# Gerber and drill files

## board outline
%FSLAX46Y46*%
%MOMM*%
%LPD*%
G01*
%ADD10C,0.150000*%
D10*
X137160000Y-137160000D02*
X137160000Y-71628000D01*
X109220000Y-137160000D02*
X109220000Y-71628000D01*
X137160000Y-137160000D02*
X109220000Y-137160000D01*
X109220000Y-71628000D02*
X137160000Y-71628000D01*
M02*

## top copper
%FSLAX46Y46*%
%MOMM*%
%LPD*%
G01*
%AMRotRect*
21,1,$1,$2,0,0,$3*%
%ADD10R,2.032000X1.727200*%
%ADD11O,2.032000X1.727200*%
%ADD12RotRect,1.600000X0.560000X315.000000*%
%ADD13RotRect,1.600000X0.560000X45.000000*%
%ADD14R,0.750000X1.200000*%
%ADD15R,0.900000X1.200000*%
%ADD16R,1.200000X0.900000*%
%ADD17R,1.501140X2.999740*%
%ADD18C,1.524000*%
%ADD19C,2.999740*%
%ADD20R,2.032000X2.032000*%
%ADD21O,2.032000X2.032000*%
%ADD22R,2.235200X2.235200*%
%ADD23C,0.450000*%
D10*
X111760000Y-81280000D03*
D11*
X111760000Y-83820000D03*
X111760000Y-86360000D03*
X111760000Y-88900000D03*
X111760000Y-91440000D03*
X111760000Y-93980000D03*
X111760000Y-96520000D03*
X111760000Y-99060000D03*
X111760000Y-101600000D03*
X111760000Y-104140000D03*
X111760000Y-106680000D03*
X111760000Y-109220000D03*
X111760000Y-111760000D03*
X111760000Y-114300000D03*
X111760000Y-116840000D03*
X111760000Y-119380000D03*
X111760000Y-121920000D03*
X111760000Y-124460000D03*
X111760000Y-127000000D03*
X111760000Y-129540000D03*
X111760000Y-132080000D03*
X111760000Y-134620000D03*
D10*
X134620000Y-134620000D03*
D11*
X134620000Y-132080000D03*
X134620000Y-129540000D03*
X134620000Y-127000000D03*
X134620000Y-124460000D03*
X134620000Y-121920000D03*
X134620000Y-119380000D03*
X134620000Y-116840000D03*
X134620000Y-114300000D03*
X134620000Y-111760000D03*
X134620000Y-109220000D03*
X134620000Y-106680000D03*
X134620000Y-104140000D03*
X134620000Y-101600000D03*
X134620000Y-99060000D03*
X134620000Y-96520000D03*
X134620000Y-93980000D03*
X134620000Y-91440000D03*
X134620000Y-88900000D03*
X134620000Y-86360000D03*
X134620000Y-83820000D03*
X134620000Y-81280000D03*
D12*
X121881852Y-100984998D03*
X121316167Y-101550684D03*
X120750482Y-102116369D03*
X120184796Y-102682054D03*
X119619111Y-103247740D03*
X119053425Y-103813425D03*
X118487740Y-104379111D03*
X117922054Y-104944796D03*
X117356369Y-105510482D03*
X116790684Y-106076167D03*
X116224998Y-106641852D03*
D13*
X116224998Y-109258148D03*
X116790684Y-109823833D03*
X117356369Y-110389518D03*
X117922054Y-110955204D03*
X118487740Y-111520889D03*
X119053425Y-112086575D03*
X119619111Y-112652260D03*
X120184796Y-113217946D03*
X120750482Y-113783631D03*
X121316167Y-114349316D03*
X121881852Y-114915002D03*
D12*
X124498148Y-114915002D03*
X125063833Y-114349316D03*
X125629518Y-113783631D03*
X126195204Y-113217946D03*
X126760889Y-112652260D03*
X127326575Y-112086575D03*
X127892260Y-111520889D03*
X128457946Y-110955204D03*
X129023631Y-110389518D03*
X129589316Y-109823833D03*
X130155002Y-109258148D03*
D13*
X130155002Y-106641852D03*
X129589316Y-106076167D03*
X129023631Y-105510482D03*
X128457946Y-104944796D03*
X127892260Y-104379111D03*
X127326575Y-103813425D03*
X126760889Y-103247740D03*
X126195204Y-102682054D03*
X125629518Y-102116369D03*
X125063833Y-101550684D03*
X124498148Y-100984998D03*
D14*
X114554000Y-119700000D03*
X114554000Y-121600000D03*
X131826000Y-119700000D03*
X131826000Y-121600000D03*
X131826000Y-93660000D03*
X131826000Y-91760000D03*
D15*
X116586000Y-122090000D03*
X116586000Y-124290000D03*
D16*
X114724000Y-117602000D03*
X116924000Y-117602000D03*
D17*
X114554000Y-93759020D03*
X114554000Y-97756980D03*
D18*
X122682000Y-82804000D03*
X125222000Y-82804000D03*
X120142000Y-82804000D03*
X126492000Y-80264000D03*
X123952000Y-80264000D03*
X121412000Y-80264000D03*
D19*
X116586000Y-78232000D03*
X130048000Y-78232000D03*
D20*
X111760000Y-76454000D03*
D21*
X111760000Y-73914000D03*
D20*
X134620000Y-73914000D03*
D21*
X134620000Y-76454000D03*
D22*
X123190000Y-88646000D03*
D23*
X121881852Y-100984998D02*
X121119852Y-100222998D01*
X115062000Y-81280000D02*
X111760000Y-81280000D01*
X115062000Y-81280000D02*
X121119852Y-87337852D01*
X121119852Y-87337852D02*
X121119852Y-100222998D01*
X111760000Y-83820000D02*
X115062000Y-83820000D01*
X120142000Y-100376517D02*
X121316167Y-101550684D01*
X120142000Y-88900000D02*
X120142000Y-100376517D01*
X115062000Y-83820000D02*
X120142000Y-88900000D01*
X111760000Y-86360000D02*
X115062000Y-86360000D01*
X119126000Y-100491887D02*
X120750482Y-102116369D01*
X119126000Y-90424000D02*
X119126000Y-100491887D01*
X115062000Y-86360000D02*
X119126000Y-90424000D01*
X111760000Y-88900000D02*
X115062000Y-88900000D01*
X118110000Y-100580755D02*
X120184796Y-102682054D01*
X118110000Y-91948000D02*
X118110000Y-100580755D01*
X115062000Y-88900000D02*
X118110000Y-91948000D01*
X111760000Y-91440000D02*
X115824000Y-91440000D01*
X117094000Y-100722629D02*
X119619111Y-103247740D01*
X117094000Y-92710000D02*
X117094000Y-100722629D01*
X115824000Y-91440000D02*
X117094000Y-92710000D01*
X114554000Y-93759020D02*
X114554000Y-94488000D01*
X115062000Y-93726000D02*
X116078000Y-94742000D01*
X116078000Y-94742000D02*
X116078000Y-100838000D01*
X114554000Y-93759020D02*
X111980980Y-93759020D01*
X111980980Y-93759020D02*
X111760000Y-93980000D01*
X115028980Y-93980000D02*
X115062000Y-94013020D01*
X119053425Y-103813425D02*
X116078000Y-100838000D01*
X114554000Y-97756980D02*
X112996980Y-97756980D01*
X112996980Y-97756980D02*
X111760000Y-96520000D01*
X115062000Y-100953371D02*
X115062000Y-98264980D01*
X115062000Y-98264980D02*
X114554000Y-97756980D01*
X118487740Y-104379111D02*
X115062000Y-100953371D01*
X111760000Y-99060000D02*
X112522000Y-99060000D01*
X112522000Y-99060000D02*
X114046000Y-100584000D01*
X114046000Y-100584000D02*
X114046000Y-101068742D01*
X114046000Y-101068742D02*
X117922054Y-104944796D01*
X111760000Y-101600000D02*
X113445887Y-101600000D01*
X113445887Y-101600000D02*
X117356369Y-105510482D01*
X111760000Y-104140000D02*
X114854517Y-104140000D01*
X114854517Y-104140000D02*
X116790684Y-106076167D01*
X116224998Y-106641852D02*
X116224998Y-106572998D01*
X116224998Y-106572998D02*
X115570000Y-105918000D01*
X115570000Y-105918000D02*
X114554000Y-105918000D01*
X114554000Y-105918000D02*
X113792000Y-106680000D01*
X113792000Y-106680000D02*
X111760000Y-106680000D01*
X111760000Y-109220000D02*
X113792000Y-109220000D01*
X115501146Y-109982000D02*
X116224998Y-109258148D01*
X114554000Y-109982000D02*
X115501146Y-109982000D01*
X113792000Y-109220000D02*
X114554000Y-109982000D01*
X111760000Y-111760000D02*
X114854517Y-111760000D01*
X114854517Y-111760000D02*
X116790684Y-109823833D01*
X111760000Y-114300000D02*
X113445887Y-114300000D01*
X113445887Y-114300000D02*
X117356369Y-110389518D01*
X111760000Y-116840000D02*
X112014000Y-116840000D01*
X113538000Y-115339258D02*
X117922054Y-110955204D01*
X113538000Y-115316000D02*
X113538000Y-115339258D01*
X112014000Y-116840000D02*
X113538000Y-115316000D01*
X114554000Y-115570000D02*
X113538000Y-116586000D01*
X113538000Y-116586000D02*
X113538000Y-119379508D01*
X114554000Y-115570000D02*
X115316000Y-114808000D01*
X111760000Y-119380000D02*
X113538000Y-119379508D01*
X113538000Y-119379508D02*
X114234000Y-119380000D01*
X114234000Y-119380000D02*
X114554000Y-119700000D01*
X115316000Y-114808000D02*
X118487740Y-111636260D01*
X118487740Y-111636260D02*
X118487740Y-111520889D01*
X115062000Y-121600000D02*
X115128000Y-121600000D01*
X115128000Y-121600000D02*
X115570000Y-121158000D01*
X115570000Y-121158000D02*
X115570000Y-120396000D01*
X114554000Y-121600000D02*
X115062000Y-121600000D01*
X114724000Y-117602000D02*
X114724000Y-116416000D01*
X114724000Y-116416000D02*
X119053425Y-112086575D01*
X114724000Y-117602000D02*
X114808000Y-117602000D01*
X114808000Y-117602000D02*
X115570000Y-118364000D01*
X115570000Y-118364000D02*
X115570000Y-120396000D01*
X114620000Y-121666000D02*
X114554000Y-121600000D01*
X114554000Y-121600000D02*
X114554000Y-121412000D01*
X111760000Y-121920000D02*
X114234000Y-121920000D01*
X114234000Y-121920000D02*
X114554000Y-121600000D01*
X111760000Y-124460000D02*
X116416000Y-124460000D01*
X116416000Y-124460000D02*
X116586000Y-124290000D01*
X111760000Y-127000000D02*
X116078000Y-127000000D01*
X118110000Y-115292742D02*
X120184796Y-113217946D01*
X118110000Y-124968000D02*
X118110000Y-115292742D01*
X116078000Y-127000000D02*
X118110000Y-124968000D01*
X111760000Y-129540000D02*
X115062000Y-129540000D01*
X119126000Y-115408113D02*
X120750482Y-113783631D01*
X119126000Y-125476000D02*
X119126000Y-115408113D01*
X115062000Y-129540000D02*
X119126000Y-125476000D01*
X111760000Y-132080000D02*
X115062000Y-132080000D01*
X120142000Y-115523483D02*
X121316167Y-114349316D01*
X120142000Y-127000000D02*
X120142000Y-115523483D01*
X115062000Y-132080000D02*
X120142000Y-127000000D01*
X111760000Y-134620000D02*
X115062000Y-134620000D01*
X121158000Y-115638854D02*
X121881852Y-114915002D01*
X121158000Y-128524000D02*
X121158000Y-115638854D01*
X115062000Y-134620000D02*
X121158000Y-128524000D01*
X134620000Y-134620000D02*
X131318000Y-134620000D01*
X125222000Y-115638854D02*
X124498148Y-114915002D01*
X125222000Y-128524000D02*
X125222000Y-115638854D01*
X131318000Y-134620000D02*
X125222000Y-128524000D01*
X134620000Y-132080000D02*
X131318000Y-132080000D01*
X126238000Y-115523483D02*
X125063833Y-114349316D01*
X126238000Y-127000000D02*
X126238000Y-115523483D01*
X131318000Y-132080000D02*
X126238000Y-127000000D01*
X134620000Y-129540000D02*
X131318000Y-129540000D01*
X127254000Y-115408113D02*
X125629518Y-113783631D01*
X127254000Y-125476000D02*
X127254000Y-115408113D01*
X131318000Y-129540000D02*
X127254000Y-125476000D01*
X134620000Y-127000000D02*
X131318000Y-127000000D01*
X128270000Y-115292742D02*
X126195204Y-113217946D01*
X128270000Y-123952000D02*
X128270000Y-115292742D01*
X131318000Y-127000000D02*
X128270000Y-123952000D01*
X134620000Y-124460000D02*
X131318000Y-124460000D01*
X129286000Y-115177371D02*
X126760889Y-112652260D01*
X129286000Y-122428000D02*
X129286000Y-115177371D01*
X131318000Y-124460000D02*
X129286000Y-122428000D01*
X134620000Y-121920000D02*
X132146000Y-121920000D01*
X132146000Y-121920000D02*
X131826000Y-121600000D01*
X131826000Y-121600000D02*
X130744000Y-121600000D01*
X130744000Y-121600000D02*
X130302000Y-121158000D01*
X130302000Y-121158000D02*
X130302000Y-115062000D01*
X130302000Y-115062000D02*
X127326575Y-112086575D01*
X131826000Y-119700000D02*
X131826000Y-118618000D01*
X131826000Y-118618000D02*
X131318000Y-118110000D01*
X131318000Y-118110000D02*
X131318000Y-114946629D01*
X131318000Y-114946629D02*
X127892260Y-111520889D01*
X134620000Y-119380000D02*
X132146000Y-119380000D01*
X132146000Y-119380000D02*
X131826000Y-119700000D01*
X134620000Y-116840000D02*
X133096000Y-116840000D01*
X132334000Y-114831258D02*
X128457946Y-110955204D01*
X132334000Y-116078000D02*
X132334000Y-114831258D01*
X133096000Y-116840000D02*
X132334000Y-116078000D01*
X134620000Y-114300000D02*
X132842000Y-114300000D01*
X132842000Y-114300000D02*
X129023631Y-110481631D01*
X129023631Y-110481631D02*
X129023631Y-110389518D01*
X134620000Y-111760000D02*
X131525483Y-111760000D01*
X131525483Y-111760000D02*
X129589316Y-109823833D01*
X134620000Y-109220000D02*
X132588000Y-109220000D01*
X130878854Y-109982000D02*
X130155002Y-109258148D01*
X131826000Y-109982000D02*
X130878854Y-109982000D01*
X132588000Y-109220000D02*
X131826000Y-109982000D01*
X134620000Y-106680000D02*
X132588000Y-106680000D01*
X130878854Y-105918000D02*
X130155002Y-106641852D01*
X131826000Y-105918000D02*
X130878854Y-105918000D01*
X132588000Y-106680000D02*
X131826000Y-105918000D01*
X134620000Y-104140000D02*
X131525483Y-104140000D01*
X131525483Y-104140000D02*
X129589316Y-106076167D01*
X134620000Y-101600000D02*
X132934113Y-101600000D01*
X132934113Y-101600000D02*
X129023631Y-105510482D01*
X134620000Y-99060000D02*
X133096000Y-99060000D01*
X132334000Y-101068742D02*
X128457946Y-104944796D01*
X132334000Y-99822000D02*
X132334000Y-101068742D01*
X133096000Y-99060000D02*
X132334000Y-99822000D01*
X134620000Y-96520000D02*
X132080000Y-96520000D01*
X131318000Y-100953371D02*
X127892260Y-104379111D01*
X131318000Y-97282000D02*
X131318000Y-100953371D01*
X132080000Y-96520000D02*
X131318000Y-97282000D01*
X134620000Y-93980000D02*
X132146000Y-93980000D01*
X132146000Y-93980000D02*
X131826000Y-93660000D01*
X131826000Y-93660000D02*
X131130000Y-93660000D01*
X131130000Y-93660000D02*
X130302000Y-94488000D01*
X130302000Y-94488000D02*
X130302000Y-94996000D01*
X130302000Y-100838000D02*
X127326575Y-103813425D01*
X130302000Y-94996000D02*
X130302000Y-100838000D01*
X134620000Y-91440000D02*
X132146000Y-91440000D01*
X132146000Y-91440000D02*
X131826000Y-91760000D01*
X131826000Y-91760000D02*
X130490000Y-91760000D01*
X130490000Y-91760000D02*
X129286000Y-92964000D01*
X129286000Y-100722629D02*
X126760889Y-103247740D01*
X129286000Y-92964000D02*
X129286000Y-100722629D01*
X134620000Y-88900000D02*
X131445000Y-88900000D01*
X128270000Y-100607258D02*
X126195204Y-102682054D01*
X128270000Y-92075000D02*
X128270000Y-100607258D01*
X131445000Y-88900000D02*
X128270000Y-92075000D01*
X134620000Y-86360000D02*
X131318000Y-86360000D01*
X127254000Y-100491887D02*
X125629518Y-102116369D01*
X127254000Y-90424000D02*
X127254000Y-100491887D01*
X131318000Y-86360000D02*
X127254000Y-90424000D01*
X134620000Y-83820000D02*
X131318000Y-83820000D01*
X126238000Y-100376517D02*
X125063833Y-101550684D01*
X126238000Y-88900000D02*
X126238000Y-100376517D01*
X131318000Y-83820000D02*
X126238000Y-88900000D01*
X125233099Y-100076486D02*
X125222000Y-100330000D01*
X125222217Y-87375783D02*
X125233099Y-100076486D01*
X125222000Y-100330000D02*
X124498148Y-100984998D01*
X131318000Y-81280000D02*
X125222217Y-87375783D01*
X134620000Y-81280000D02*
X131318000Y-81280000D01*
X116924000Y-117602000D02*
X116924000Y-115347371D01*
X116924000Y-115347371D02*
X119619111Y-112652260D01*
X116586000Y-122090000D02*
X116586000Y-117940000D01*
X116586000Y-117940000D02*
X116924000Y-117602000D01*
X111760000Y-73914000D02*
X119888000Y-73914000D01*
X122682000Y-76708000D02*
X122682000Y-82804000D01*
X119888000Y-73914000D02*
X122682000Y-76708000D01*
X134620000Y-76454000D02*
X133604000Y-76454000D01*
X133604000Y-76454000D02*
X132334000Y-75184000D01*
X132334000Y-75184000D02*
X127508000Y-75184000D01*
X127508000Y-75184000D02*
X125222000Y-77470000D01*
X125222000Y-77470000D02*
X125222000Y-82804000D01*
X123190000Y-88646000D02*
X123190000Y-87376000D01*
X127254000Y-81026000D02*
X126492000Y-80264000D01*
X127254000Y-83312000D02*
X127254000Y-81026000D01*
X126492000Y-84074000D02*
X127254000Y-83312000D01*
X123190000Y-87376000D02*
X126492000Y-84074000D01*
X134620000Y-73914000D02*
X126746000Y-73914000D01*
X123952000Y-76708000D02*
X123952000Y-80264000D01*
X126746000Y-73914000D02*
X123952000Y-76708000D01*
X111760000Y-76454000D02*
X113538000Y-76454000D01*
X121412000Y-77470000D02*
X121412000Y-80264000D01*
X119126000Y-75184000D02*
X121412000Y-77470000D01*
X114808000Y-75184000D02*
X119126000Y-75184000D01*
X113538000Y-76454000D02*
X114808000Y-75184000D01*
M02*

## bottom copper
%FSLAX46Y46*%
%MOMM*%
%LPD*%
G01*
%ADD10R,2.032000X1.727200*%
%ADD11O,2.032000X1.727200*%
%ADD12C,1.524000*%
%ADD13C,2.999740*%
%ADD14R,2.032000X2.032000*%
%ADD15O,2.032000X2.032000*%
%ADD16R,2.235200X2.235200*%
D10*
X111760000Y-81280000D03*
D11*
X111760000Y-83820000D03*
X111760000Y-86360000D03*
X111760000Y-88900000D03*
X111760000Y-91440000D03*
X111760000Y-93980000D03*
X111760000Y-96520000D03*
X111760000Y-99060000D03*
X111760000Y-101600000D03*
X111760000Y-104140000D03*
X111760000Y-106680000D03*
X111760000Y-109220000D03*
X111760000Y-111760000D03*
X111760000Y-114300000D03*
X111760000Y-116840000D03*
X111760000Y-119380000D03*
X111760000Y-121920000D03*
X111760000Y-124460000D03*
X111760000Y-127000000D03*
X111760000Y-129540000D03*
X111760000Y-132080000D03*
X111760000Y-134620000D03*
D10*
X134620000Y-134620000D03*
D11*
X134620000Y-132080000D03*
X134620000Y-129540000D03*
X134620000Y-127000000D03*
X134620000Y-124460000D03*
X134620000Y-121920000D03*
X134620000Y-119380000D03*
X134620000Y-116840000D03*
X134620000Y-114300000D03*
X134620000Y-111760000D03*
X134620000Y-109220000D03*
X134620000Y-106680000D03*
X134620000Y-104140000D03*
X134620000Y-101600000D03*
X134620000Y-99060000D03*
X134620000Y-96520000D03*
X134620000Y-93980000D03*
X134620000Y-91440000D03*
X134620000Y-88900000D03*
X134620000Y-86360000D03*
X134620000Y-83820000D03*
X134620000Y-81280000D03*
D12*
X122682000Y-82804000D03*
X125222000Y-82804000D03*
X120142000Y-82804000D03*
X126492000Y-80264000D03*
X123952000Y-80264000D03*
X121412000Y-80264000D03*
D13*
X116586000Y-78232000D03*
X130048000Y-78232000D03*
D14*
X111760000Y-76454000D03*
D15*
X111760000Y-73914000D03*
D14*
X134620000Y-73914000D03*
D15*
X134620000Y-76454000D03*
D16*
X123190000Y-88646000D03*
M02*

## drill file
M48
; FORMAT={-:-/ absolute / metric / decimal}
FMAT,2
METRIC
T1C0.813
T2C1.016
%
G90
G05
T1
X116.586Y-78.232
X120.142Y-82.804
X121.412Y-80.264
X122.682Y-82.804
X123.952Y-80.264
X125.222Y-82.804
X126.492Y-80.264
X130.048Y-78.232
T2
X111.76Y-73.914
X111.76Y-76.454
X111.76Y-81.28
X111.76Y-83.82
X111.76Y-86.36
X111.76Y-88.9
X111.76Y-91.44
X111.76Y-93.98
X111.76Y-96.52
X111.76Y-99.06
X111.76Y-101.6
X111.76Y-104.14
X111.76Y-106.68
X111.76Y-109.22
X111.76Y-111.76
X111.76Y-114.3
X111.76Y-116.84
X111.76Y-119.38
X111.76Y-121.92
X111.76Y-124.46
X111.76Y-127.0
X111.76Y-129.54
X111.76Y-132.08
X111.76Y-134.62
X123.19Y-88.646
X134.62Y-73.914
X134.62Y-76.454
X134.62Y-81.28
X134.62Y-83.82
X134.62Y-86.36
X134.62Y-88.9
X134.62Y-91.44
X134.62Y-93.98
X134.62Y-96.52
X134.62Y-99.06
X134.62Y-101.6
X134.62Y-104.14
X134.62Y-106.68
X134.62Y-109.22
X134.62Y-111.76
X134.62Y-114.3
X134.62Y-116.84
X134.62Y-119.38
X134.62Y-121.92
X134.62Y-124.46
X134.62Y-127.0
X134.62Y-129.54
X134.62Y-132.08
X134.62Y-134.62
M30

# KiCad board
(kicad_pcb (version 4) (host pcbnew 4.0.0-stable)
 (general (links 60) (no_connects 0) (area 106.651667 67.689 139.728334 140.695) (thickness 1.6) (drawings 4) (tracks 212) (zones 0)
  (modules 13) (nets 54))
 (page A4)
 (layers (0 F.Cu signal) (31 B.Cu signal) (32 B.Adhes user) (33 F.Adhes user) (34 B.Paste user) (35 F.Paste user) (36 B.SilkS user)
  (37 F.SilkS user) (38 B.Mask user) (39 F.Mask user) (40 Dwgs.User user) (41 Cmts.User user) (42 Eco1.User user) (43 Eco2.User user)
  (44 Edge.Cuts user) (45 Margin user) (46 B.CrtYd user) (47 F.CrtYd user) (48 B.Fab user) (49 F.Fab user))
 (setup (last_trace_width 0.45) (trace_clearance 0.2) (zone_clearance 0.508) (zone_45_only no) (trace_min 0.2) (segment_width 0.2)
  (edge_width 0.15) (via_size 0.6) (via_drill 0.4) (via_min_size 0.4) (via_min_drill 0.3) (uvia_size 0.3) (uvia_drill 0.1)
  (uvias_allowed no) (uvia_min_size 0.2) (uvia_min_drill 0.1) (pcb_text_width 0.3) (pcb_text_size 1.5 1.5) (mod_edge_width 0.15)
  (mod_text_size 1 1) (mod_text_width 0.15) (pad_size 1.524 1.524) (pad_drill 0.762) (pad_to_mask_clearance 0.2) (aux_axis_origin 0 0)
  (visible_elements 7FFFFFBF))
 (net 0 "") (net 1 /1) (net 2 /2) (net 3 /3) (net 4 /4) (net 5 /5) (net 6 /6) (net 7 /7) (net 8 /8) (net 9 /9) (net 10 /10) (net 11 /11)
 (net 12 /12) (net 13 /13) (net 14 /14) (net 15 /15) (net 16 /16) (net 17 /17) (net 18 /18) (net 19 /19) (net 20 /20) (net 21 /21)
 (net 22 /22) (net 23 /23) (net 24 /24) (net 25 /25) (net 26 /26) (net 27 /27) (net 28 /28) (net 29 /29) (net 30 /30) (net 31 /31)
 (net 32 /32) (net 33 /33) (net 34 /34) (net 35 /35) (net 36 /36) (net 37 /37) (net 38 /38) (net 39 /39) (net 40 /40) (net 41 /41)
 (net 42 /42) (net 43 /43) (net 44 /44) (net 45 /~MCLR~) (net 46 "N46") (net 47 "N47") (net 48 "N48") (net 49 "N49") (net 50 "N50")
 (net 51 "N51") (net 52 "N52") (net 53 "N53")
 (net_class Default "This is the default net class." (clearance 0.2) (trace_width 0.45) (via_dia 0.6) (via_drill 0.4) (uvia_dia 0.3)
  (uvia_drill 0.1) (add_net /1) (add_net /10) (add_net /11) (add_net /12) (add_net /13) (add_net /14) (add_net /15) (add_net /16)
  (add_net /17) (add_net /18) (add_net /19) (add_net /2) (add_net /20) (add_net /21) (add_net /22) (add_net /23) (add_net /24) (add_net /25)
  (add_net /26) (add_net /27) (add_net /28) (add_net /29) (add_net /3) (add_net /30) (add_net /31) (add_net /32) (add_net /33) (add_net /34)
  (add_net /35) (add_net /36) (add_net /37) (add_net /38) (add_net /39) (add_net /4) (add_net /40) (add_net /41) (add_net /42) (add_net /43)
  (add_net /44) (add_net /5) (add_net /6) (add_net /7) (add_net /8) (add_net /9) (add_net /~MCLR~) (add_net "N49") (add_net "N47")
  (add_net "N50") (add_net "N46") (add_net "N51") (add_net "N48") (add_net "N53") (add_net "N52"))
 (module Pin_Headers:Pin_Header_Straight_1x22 (layer B.Cu) (at 111.76 81.28 180)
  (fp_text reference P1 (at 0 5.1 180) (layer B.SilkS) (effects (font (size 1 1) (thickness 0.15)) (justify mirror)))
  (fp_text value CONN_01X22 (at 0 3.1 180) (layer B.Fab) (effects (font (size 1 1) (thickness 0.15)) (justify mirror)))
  (pad 1 thru_hole rect (at 0 0 180) (size 2.032 1.7272) (drill 1.016) (layers *.Cu *.Mask B.SilkS) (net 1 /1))
  (pad 2 thru_hole oval (at 0 -2.54 180) (size 2.032 1.7272) (drill 1.016) (layers *.Cu *.Mask B.SilkS) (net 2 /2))
  (pad 3 thru_hole oval (at 0 -5.08 180) (size 2.032 1.7272) (drill 1.016) (layers *.Cu *.Mask B.SilkS) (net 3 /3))
  (pad 4 thru_hole oval (at 0 -7.62 180) (size 2.032 1.7272) (drill 1.016) (layers *.Cu *.Mask B.SilkS) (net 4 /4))
  (pad 5 thru_hole oval (at 0 -10.16 180) (size 2.032 1.7272) (drill 1.016) (layers *.Cu *.Mask B.SilkS) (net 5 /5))
  (pad 6 thru_hole oval (at 0 -12.7 180) (size 2.032 1.7272) (drill 1.016) (layers *.Cu *.Mask B.SilkS) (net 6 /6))
  (pad 7 thru_hole oval (at 0 -15.24 180) (size 2.032 1.7272) (drill 1.016) (layers *.Cu *.Mask B.SilkS) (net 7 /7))
  (pad 8 thru_hole oval (at 0 -17.78 180) (size 2.032 1.7272) (drill 1.016) (layers *.Cu *.Mask B.SilkS) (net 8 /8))
  (pad 9 thru_hole oval (at 0 -20.32 180) (size 2.032 1.7272) (drill 1.016) (layers *.Cu *.Mask B.SilkS) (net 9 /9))
  (pad 10 thru_hole oval (at 0 -22.86 180) (size 2.032 1.7272) (drill 1.016) (layers *.Cu *.Mask B.SilkS) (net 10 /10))
  (pad 11 thru_hole oval (at 0 -25.4 180) (size 2.032 1.7272) (drill 1.016) (layers *.Cu *.Mask B.SilkS) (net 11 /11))
  (pad 12 thru_hole oval (at 0 -27.94 180) (size 2.032 1.7272) (drill 1.016) (layers *.Cu *.Mask B.SilkS) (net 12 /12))
  (pad 13 thru_hole oval (at 0 -30.48 180) (size 2.032 1.7272) (drill 1.016) (layers *.Cu *.Mask B.SilkS) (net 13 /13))
  (pad 14 thru_hole oval (at 0 -33.02 180) (size 2.032 1.7272) (drill 1.016) (layers *.Cu *.Mask B.SilkS) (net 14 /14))
  (pad 15 thru_hole oval (at 0 -35.56 180) (size 2.032 1.7272) (drill 1.016) (layers *.Cu *.Mask B.SilkS) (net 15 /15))
  (pad 16 thru_hole oval (at 0 -38.1 180) (size 2.032 1.7272) (drill 1.016) (layers *.Cu *.Mask B.SilkS) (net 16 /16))
  (pad 17 thru_hole oval (at 0 -40.64 180) (size 2.032 1.7272) (drill 1.016) (layers *.Cu *.Mask B.SilkS) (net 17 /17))
  (pad 18 thru_hole oval (at 0 -43.18 180) (size 2.032 1.7272) (drill 1.016) (layers *.Cu *.Mask B.SilkS) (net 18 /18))
  (pad 19 thru_hole oval (at 0 -45.72 180) (size 2.032 1.7272) (drill 1.016) (layers *.Cu *.Mask B.SilkS) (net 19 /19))
  (pad 20 thru_hole oval (at 0 -48.26 180) (size 2.032 1.7272) (drill 1.016) (layers *.Cu *.Mask B.SilkS) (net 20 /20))
  (pad 21 thru_hole oval (at 0 -50.8 180) (size 2.032 1.7272) (drill 1.016) (layers *.Cu *.Mask B.SilkS) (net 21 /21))
  (pad 22 thru_hole oval (at 0 -53.34 180) (size 2.032 1.7272) (drill 1.016) (layers *.Cu *.Mask B.SilkS) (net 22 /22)))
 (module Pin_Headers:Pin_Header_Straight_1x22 (layer B.Cu) (at 134.62 134.62)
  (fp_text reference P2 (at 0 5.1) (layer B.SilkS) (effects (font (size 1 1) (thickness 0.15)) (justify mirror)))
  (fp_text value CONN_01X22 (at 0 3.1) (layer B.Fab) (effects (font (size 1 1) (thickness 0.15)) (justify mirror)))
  (pad 1 thru_hole rect (at 0 0) (size 2.032 1.7272) (drill 1.016) (layers *.Cu *.Mask B.SilkS) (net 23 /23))
  (pad 2 thru_hole oval (at 0 -2.54) (size 2.032 1.7272) (drill 1.016) (layers *.Cu *.Mask B.SilkS) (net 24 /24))
  (pad 3 thru_hole oval (at 0 -5.08) (size 2.032 1.7272) (drill 1.016) (layers *.Cu *.Mask B.SilkS) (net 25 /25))
  (pad 4 thru_hole oval (at 0 -7.62) (size 2.032 1.7272) (drill 1.016) (layers *.Cu *.Mask B.SilkS) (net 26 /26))
  (pad 5 thru_hole oval (at 0 -10.16) (size 2.032 1.7272) (drill 1.016) (layers *.Cu *.Mask B.SilkS) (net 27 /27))
  (pad 6 thru_hole oval (at 0 -12.7) (size 2.032 1.7272) (drill 1.016) (layers *.Cu *.Mask B.SilkS) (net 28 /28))
  (pad 7 thru_hole oval (at 0 -15.24) (size 2.032 1.7272) (drill 1.016) (layers *.Cu *.Mask B.SilkS) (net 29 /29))
  (pad 8 thru_hole oval (at 0 -17.78) (size 2.032 1.7272) (drill 1.016) (layers *.Cu *.Mask B.SilkS) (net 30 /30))
  (pad 9 thru_hole oval (at 0 -20.32) (size 2.032 1.7272) (drill 1.016) (layers *.Cu *.Mask B.SilkS) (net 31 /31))
  (pad 10 thru_hole oval (at 0 -22.86) (size 2.032 1.7272) (drill 1.016) (layers *.Cu *.Mask B.SilkS) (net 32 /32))
  (pad 11 thru_hole oval (at 0 -25.4) (size 2.032 1.7272) (drill 1.016) (layers *.Cu *.Mask B.SilkS) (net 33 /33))
  (pad 12 thru_hole oval (at 0 -27.94) (size 2.032 1.7272) (drill 1.016) (layers *.Cu *.Mask B.SilkS) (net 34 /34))
  (pad 13 thru_hole oval (at 0 -30.48) (size 2.032 1.7272) (drill 1.016) (layers *.Cu *.Mask B.SilkS) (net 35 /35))
  (pad 14 thru_hole oval (at 0 -33.02) (size 2.032 1.7272) (drill 1.016) (layers *.Cu *.Mask B.SilkS) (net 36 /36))
  (pad 15 thru_hole oval (at 0 -35.56) (size 2.032 1.7272) (drill 1.016) (layers *.Cu *.Mask B.SilkS) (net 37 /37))
  (pad 16 thru_hole oval (at 0 -38.1) (size 2.032 1.7272) (drill 1.016) (layers *.Cu *.Mask B.SilkS) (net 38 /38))
  (pad 17 thru_hole oval (at 0 -40.64) (size 2.032 1.7272) (drill 1.016) (layers *.Cu *.Mask B.SilkS) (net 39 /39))
  (pad 18 thru_hole oval (at 0 -43.18) (size 2.032 1.7272) (drill 1.016) (layers *.Cu *.Mask B.SilkS) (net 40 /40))
  (pad 19 thru_hole oval (at 0 -45.72) (size 2.032 1.7272) (drill 1.016) (layers *.Cu *.Mask B.SilkS) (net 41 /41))
  (pad 20 thru_hole oval (at 0 -48.26) (size 2.032 1.7272) (drill 1.016) (layers *.Cu *.Mask B.SilkS) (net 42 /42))
  (pad 21 thru_hole oval (at 0 -50.8) (size 2.032 1.7272) (drill 1.016) (layers *.Cu *.Mask B.SilkS) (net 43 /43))
  (pad 22 thru_hole oval (at 0 -53.34) (size 2.032 1.7272) (drill 1.016) (layers *.Cu *.Mask B.SilkS) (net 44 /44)))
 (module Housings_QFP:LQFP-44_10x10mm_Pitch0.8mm (layer F.Cu) (at 123.19 107.95 315)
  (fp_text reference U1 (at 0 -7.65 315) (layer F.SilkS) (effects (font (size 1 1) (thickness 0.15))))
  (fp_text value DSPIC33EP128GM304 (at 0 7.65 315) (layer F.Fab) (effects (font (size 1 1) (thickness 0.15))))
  (pad 1 smd rect (at -5.85 -4 315) (size 1.6 0.56) (layers F.Cu F.Paste F.Mask) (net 1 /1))
  (pad 2 smd rect (at -5.85 -3.2 315) (size 1.6 0.56) (layers F.Cu F.Paste F.Mask) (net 2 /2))
  (pad 3 smd rect (at -5.85 -2.4 315) (size 1.6 0.56) (layers F.Cu F.Paste F.Mask) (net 3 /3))
  (pad 4 smd rect (at -5.85 -1.6 315) (size 1.6 0.56) (layers F.Cu F.Paste F.Mask) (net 4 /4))
  (pad 5 smd rect (at -5.85 -0.8 315) (size 1.6 0.56) (layers F.Cu F.Paste F.Mask) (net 5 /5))
  (pad 6 smd rect (at -5.85 0 315) (size 1.6 0.56) (layers F.Cu F.Paste F.Mask) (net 6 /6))
  (pad 7 smd rect (at -5.85 0.8 315) (size 1.6 0.56) (layers F.Cu F.Paste F.Mask) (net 7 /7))
  (pad 8 smd rect (at -5.85 1.6 315) (size 1.6 0.56) (layers F.Cu F.Paste F.Mask) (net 8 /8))
  (pad 9 smd rect (at -5.85 2.4 315) (size 1.6 0.56) (layers F.Cu F.Paste F.Mask) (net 9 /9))
  (pad 10 smd rect (at -5.85 3.2 315) (size 1.6 0.56) (layers F.Cu F.Paste F.Mask) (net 10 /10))
  (pad 11 smd rect (at -5.85 4 315) (size 1.6 0.56) (layers F.Cu F.Paste F.Mask) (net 11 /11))
  (pad 12 smd rect (at -4 5.85 45) (size 1.6 0.56) (layers F.Cu F.Paste F.Mask) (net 12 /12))
  (pad 13 smd rect (at -3.2 5.85 45) (size 1.6 0.56) (layers F.Cu F.Paste F.Mask) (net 13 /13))
  (pad 14 smd rect (at -2.4 5.85 45) (size 1.6 0.56) (layers F.Cu F.Paste F.Mask) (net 14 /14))
  (pad 15 smd rect (at -1.6 5.85 45) (size 1.6 0.56) (layers F.Cu F.Paste F.Mask) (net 15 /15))
  (pad 16 smd rect (at -0.8 5.85 45) (size 1.6 0.56) (layers F.Cu F.Paste F.Mask) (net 16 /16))
  (pad 17 smd rect (at 0 5.85 45) (size 1.6 0.56) (layers F.Cu F.Paste F.Mask) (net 17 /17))
  (pad 18 smd rect (at 0.8 5.85 45) (size 1.6 0.56) (layers F.Cu F.Paste F.Mask) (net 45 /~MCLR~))
  (pad 19 smd rect (at 1.6 5.85 45) (size 1.6 0.56) (layers F.Cu F.Paste F.Mask) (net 19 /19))
  (pad 20 smd rect (at 2.4 5.85 45) (size 1.6 0.56) (layers F.Cu F.Paste F.Mask) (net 20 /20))
  (pad 21 smd rect (at 3.2 5.85 45) (size 1.6 0.56) (layers F.Cu F.Paste F.Mask) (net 21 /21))
  (pad 22 smd rect (at 4 5.85 45) (size 1.6 0.56) (layers F.Cu F.Paste F.Mask) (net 22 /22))
  (pad 23 smd rect (at 5.85 4 315) (size 1.6 0.56) (layers F.Cu F.Paste F.Mask) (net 23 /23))
  (pad 24 smd rect (at 5.85 3.2 315) (size 1.6 0.56) (layers F.Cu F.Paste F.Mask) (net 24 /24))
  (pad 25 smd rect (at 5.85 2.4 315) (size 1.6 0.56) (layers F.Cu F.Paste F.Mask) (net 25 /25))
  (pad 26 smd rect (at 5.85 1.6 315) (size 1.6 0.56) (layers F.Cu F.Paste F.Mask) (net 26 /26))
  (pad 27 smd rect (at 5.85 0.8 315) (size 1.6 0.56) (layers F.Cu F.Paste F.Mask) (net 27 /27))
  (pad 28 smd rect (at 5.85 0 315) (size 1.6 0.56) (layers F.Cu F.Paste F.Mask) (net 28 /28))
  (pad 29 smd rect (at 5.85 -0.8 315) (size 1.6 0.56) (layers F.Cu F.Paste F.Mask) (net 29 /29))
  (pad 30 smd rect (at 5.85 -1.6 315) (size 1.6 0.56) (layers F.Cu F.Paste F.Mask) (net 30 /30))
  (pad 31 smd rect (at 5.85 -2.4 315) (size 1.6 0.56) (layers F.Cu F.Paste F.Mask) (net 31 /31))
  (pad 32 smd rect (at 5.85 -3.2 315) (size 1.6 0.56) (layers F.Cu F.Paste F.Mask) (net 32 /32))
  (pad 33 smd rect (at 5.85 -4 315) (size 1.6 0.56) (layers F.Cu F.Paste F.Mask) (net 33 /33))
  (pad 34 smd rect (at 4 -5.85 45) (size 1.6 0.56) (layers F.Cu F.Paste F.Mask) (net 34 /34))
  (pad 35 smd rect (at 3.2 -5.85 45) (size 1.6 0.56) (layers F.Cu F.Paste F.Mask) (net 35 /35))
  (pad 36 smd rect (at 2.4 -5.85 45) (size 1.6 0.56) (layers F.Cu F.Paste F.Mask) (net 36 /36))
  (pad 37 smd rect (at 1.6 -5.85 45) (size 1.6 0.56) (layers F.Cu F.Paste F.Mask) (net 37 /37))
  (pad 38 smd rect (at 0.8 -5.85 45) (size 1.6 0.56) (layers F.Cu F.Paste F.Mask) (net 38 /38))
  (pad 39 smd rect (at 0 -5.85 45) (size 1.6 0.56) (layers F.Cu F.Paste F.Mask) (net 39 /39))
  (pad 40 smd rect (at -0.8 -5.85 45) (size 1.6 0.56) (layers F.Cu F.Paste F.Mask) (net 40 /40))
  (pad 41 smd rect (at -1.6 -5.85 45) (size 1.6 0.56) (layers F.Cu F.Paste F.Mask) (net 41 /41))
  (pad 42 smd rect (at -2.4 -5.85 45) (size 1.6 0.56) (layers F.Cu F.Paste F.Mask) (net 42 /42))
  (pad 43 smd rect (at -3.2 -5.85 45) (size 1.6 0.56) (layers F.Cu F.Paste F.Mask) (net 43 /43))
  (pad 44 smd rect (at -4 -5.85 45) (size 1.6 0.56) (layers F.Cu F.Paste F.Mask) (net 44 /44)))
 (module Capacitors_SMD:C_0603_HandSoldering (layer F.Cu) (at 114.554 120.65 270)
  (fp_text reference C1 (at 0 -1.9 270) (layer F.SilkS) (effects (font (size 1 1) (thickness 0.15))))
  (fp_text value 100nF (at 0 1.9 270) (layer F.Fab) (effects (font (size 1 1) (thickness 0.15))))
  (pad 1 smd rect (at -0.95 0 270) (size 1.2 0.75) (layers F.Cu F.Paste F.Mask) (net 16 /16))
  (pad 2 smd rect (at 0.95 0 270) (size 1.2 0.75) (layers F.Cu F.Paste F.Mask) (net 17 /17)))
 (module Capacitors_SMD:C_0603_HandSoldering (layer F.Cu) (at 131.826 120.65 270)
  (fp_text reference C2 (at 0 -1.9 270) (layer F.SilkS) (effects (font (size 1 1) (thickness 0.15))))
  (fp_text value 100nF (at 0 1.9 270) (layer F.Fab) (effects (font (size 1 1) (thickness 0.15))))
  (pad 1 smd rect (at -0.95 0 270) (size 1.2 0.75) (layers F.Cu F.Paste F.Mask) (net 29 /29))
  (pad 2 smd rect (at 0.95 0 270) (size 1.2 0.75) (layers F.Cu F.Paste F.Mask) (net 28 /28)))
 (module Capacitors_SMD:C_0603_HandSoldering (layer F.Cu) (at 131.826 92.71 90)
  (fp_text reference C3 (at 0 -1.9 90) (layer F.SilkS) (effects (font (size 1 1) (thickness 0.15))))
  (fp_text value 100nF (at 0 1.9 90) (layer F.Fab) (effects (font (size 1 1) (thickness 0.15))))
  (pad 1 smd rect (at -0.95 0 90) (size 1.2 0.75) (layers F.Cu F.Paste F.Mask) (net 39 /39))
  (pad 2 smd rect (at 0.95 0 90) (size 1.2 0.75) (layers F.Cu F.Paste F.Mask) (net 40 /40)))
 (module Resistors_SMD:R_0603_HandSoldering (layer F.Cu) (at 116.586 123.19 270)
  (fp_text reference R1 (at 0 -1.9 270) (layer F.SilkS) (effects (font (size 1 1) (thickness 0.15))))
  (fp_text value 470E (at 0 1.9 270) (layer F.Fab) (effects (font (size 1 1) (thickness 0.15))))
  (pad 1 smd rect (at -1.1 0 270) (size 1.2 0.9) (layers F.Cu F.Paste F.Mask) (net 45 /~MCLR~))
  (pad 2 smd rect (at 1.1 0 270) (size 1.2 0.9) (layers F.Cu F.Paste F.Mask) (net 18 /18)))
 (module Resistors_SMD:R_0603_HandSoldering (layer F.Cu) (at 115.824 117.602)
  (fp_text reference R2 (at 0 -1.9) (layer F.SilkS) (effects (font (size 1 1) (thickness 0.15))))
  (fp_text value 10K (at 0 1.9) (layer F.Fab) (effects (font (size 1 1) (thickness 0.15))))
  (pad 1 smd rect (at -1.1 0) (size 1.2 0.9) (layers F.Cu F.Paste F.Mask) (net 17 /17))
  (pad 2 smd rect (at 1.1 0) (size 1.2 0.9) (layers F.Cu F.Paste F.Mask) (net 45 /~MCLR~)))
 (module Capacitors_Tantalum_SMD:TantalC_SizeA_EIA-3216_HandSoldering (layer F.Cu) (at 114.554 95.758 90)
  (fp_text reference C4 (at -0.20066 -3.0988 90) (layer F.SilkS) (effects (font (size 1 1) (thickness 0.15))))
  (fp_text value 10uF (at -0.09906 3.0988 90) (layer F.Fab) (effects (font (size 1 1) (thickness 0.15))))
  (pad 2 smd rect (at 1.99898 0 90) (size 2.99974 1.50114) (layers F.Cu F.Paste F.Mask) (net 6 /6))
  (pad 1 smd rect (at -1.99898 0 90) (size 2.99974 1.50114) (layers F.Cu F.Paste F.Mask) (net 7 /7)))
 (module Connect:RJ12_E (layer F.Cu) (at 123.19 73.914 180)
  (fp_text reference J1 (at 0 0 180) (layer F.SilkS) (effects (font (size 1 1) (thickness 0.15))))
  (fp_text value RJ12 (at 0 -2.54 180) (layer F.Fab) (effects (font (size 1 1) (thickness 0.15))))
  (pad 4 thru_hole circle (at 0.508 -8.89 180) (size 1.524 1.524) (drill 0.8128) (layers *.Cu *.Mask F.SilkS) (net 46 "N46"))
  (pad 2 thru_hole circle (at -2.032 -8.89 180) (size 1.524 1.524) (drill 0.8128) (layers *.Cu *.Mask F.SilkS) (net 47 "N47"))
  (pad 6 thru_hole circle (at 3.048 -8.89 180) (size 1.524 1.524) (drill 0.8128) (layers *.Cu *.Mask F.SilkS) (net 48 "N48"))
  (pad 1 thru_hole circle (at -3.302 -6.35 180) (size 1.524 1.524) (drill 0.8128) (layers *.Cu *.Mask F.SilkS) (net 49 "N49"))
  (pad 3 thru_hole circle (at -0.762 -6.35 180) (size 1.524 1.524) (drill 0.8128) (layers *.Cu *.Mask F.SilkS) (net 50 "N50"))
  (pad 5 thru_hole circle (at 1.778 -6.35 180) (size 1.524 1.524) (drill 0.8128) (layers *.Cu *.Mask F.SilkS) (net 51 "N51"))
  (pad 8 thru_hole circle (at 6.604 -4.318 180) (size 2.99974 2.99974) (drill 0.8128) (layers *.Cu *.Mask F.SilkS) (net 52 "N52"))
  (pad 7 thru_hole circle (at -6.858 -4.318 180) (size 2.99974 2.99974) (drill 0.8128) (layers *.Cu *.Mask F.SilkS) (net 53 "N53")))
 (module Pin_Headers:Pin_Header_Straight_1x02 (layer F.Cu) (at 111.76 76.454 180)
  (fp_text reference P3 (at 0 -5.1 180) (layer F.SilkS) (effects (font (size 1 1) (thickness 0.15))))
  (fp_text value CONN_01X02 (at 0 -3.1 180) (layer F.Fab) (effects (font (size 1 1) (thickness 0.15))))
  (pad 1 thru_hole rect (at 0 0 180) (size 2.032 2.032) (drill 1.016) (layers *.Cu *.Mask F.SilkS) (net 51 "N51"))
  (pad 2 thru_hole oval (at 0 2.54 180) (size 2.032 2.032) (drill 1.016) (layers *.Cu *.Mask F.SilkS) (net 46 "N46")))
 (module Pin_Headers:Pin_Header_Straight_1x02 (layer F.Cu) (at 134.62 73.914)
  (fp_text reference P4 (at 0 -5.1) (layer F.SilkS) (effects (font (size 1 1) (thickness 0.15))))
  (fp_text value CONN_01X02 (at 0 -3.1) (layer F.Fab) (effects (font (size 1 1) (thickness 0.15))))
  (pad 1 thru_hole rect (at 0 0) (size 2.032 2.032) (drill 1.016) (layers *.Cu *.Mask F.SilkS) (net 50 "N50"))
  (pad 2 thru_hole oval (at 0 2.54) (size 2.032 2.032) (drill 1.016) (layers *.Cu *.Mask F.SilkS) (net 47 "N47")))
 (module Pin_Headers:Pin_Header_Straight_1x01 (layer F.Cu) (at 123.19 88.646)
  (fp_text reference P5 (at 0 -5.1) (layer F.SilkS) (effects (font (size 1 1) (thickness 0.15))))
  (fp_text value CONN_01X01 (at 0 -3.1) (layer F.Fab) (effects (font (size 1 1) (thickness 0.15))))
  (pad 1 thru_hole rect (at 0 0) (size 2.2352 2.2352) (drill 1.016) (layers *.Cu *.Mask F.SilkS) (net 49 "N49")))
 (gr_line (start 137.16 137.16) (end 137.16 71.628) (angle 90) (layer Edge.Cuts) (width 0.15))
 (gr_line (start 109.22 137.16) (end 109.22 71.628) (angle 90) (layer Edge.Cuts) (width 0.15))
 (gr_line (start 137.16 137.16) (end 109.22 137.16) (angle 90) (layer Edge.Cuts) (width 0.15))
 (gr_line (start 109.22 71.628) (end 137.16 71.628) (angle 90) (layer Edge.Cuts) (width 0.15))
 (segment (start 121.881852 100.984998) (end 121.119852 100.222998) (width 0.45) (layer F.Cu) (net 1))
 (segment (start 115.062 81.28) (end 111.76 81.28) (width 0.45) (layer F.Cu) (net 1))
 (segment (start 115.062 81.28) (end 121.119852 87.337852) (width 0.45) (layer F.Cu) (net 1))
 (segment (start 121.119852 87.337852) (end 121.119852 100.222998) (width 0.45) (layer F.Cu) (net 1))
 (segment (start 111.76 83.82) (end 115.062 83.82) (width 0.45) (layer F.Cu) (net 2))
 (segment (start 120.142 100.376517) (end 121.316167 101.550684) (width 0.45) (layer F.Cu) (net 2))
 (segment (start 120.142 88.9) (end 120.142 100.376517) (width 0.45) (layer F.Cu) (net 2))
 (segment (start 115.062 83.82) (end 120.142 88.9) (width 0.45) (layer F.Cu) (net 2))
 (segment (start 111.76 86.36) (end 115.062 86.36) (width 0.45) (layer F.Cu) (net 3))
 (segment (start 119.126 100.491887) (end 120.750482 102.116369) (width 0.45) (layer F.Cu) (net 3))
 (segment (start 119.126 90.424) (end 119.126 100.491887) (width 0.45) (layer F.Cu) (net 3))
 (segment (start 115.062 86.36) (end 119.126 90.424) (width 0.45) (layer F.Cu) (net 3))
 (segment (start 111.76 88.9) (end 115.062 88.9) (width 0.45) (layer F.Cu) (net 4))
 (segment (start 118.11 100.580755) (end 120.184796 102.682054) (width 0.45) (layer F.Cu) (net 4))
 (segment (start 118.11 91.948) (end 118.11 100.580755) (width 0.45) (layer F.Cu) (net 4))
 (segment (start 115.062 88.9) (end 118.11 91.948) (width 0.45) (layer F.Cu) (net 4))
 (segment (start 111.76 91.44) (end 115.824 91.44) (width 0.45) (layer F.Cu) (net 5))
 (segment (start 117.094 100.722629) (end 119.619111 103.24774) (width 0.45) (layer F.Cu) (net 5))
 (segment (start 117.094 92.71) (end 117.094 100.722629) (width 0.45) (layer F.Cu) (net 5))
 (segment (start 115.824 91.44) (end 117.094 92.71) (width 0.45) (layer F.Cu) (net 5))
 (segment (start 114.554 93.75902) (end 114.554 94.488) (width 0.45) (layer F.Cu) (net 6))
 (segment (start 115.062 93.726) (end 116.078 94.742) (width 0.45) (layer F.Cu) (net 6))
 (segment (start 116.078 94.742) (end 116.078 100.838) (width 0.45) (layer F.Cu) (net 6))
 (segment (start 114.554 93.75902) (end 111.98098 93.75902) (width 0.45) (layer F.Cu) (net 6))
 (segment (start 111.98098 93.75902) (end 111.76 93.98) (width 0.45) (layer F.Cu) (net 6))
 (segment (start 115.02898 93.98) (end 115.062 94.01302) (width 0.45) (layer F.Cu) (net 6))
 (segment (start 119.053425 103.813425) (end 116.078 100.838) (width 0.45) (layer F.Cu) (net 6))
 (segment (start 114.554 97.75698) (end 112.99698 97.75698) (width 0.45) (layer F.Cu) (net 7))
 (segment (start 112.99698 97.75698) (end 111.76 96.52) (width 0.45) (layer F.Cu) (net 7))
 (segment (start 115.062 100.953371) (end 115.062 98.26498) (width 0.45) (layer F.Cu) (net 7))
 (segment (start 115.062 98.26498) (end 114.554 97.75698) (width 0.45) (layer F.Cu) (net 7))
 (segment (start 118.48774 104.379111) (end 115.062 100.953371) (width 0.45) (layer F.Cu) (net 7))
 (segment (start 111.76 99.06) (end 112.522 99.06) (width 0.45) (layer F.Cu) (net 8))
 (segment (start 112.522 99.06) (end 114.046 100.584) (width 0.45) (layer F.Cu) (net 8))
 (segment (start 114.046 100.584) (end 114.046 101.068742) (width 0.45) (layer F.Cu) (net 8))
 (segment (start 114.046 101.068742) (end 117.922054 104.944796) (width 0.45) (layer F.Cu) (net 8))
 (segment (start 111.76 101.6) (end 113.445887 101.6) (width 0.45) (layer F.Cu) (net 9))
 (segment (start 113.445887 101.6) (end 117.356369 105.510482) (width 0.45) (layer F.Cu) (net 9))
 (segment (start 111.76 104.14) (end 114.854517 104.14) (width 0.45) (layer F.Cu) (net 10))
 (segment (start 114.854517 104.14) (end 116.790684 106.076167) (width 0.45) (layer F.Cu) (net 10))
 (segment (start 116.224998 106.641852) (end 116.224998 106.572998) (width 0.45) (layer F.Cu) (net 11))
 (segment (start 116.224998 106.572998) (end 115.57 105.918) (width 0.45) (layer F.Cu) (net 11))
 (segment (start 115.57 105.918) (end 114.554 105.918) (width 0.45) (layer F.Cu) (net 11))
 (segment (start 114.554 105.918) (end 113.792 106.68) (width 0.45) (layer F.Cu) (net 11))
 (segment (start 113.792 106.68) (end 111.76 106.68) (width 0.45) (layer F.Cu) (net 11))
 (segment (start 111.76 109.22) (end 113.792 109.22) (width 0.45) (layer F.Cu) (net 12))
 (segment (start 115.501146 109.982) (end 116.224998 109.258148) (width 0.45) (layer F.Cu) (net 12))
 (segment (start 114.554 109.982) (end 115.501146 109.982) (width 0.45) (layer F.Cu) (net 12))
 (segment (start 113.792 109.22) (end 114.554 109.982) (width 0.45) (layer F.Cu) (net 12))
 (segment (start 111.76 111.76) (end 114.854517 111.76) (width 0.45) (layer F.Cu) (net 13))
 (segment (start 114.854517 111.76) (end 116.790684 109.823833) (width 0.45) (layer F.Cu) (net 13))
 (segment (start 111.76 114.3) (end 113.445887 114.3) (width 0.45) (layer F.Cu) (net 14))
 (segment (start 113.445887 114.3) (end 117.356369 110.389518) (width 0.45) (layer F.Cu) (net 14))
 (segment (start 111.76 116.84) (end 112.014 116.84) (width 0.45) (layer F.Cu) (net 15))
 (segment (start 113.538 115.339258) (end 117.922054 110.955204) (width 0.45) (layer F.Cu) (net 15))
 (segment (start 113.538 115.316) (end 113.538 115.339258) (width 0.45) (layer F.Cu) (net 15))
 (segment (start 112.014 116.84) (end 113.538 115.316) (width 0.45) (layer F.Cu) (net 15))
 (segment (start 114.554 115.57) (end 113.538 116.586) (width 0.45) (layer F.Cu) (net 16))
 (segment (start 113.538 116.586) (end 113.538 119.379508) (width 0.45) (layer F.Cu) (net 16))
 (segment (start 114.554 115.57) (end 115.316 114.808) (width 0.45) (layer F.Cu) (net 16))
 (segment (start 111.76 119.38) (end 113.538 119.379508) (width 0.45) (layer F.Cu) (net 16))
 (segment (start 113.538 119.379508) (end 114.234 119.38) (width 0.45) (layer F.Cu) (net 16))
 (segment (start 114.234 119.38) (end 114.554 119.7) (width 0.45) (layer F.Cu) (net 16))
 (segment (start 115.316 114.808) (end 118.48774 111.63626) (width 0.45) (layer F.Cu) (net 16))
 (segment (start 118.48774 111.63626) (end 118.48774 111.520889) (width 0.45) (layer F.Cu) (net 16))
 (segment (start 115.062 121.6) (end 115.128 121.6) (width 0.45) (layer F.Cu) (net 17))
 (segment (start 115.128 121.6) (end 115.57 121.158) (width 0.45) (layer F.Cu) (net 17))
 (segment (start 115.57 121.158) (end 115.57 120.396) (width 0.45) (layer F.Cu) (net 17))
 (segment (start 114.554 121.6) (end 115.062 121.6) (width 0.45) (layer F.Cu) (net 17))
 (segment (start 114.724 117.602) (end 114.724 116.416) (width 0.45) (layer F.Cu) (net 17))
 (segment (start 114.724 116.416) (end 119.053425 112.086575) (width 0.45) (layer F.Cu) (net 17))
 (segment (start 114.724 117.602) (end 114.808 117.602) (width 0.45) (layer F.Cu) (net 17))
 (segment (start 114.808 117.602) (end 115.57 118.364) (width 0.45) (layer F.Cu) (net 17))
 (segment (start 115.57 118.364) (end 115.57 120.396) (width 0.45) (layer F.Cu) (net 17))
 (segment (start 114.62 121.666) (end 114.554 121.6) (width 0.45) (layer F.Cu) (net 17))
 (segment (start 114.554 121.6) (end 114.554 121.412) (width 0.45) (layer F.Cu) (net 17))
 (segment (start 111.76 121.92) (end 114.234 121.92) (width 0.45) (layer F.Cu) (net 17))
 (segment (start 114.234 121.92) (end 114.554 121.6) (width 0.45) (layer F.Cu) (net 17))
 (segment (start 111.76 124.46) (end 116.416 124.46) (width 0.45) (layer F.Cu) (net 18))
 (segment (start 116.416 124.46) (end 116.586 124.29) (width 0.45) (layer F.Cu) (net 18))
 (segment (start 111.76 127) (end 116.078 127) (width 0.45) (layer F.Cu) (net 19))
 (segment (start 118.11 115.292742) (end 120.184796 113.217946) (width 0.45) (layer F.Cu) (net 19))
 (segment (start 118.11 124.968) (end 118.11 115.292742) (width 0.45) (layer F.Cu) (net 19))
 (segment (start 116.078 127) (end 118.11 124.968) (width 0.45) (layer F.Cu) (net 19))
 (segment (start 111.76 129.54) (end 115.062 129.54) (width 0.45) (layer F.Cu) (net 20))
 (segment (start 119.126 115.408113) (end 120.750482 113.783631) (width 0.45) (layer F.Cu) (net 20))
 (segment (start 119.126 125.476) (end 119.126 115.408113) (width 0.45) (layer F.Cu) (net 20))
 (segment (start 115.062 129.54) (end 119.126 125.476) (width 0.45) (layer F.Cu) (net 20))
 (segment (start 111.76 132.08) (end 115.062 132.08) (width 0.45) (layer F.Cu) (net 21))
 (segment (start 120.142 115.523483) (end 121.316167 114.349316) (width 0.45) (layer F.Cu) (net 21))
 (segment (start 120.142 127) (end 120.142 115.523483) (width 0.45) (layer F.Cu) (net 21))
 (segment (start 115.062 132.08) (end 120.142 127) (width 0.45) (layer F.Cu) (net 21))
 (segment (start 111.76 134.62) (end 115.062 134.62) (width 0.45) (layer F.Cu) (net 22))
 (segment (start 121.158 115.638854) (end 121.881852 114.915002) (width 0.45) (layer F.Cu) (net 22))
 (segment (start 121.158 128.524) (end 121.158 115.638854) (width 0.45) (layer F.Cu) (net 22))
 (segment (start 115.062 134.62) (end 121.158 128.524) (width 0.45) (layer F.Cu) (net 22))
 (segment (start 134.62 134.62) (end 131.318 134.62) (width 0.45) (layer F.Cu) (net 23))
 (segment (start 125.222 115.638854) (end 124.498148 114.915002) (width 0.45) (layer F.Cu) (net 23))
 (segment (start 125.222 128.524) (end 125.222 115.638854) (width 0.45) (layer F.Cu) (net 23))
 (segment (start 131.318 134.62) (end 125.222 128.524) (width 0.45) (layer F.Cu) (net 23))
 (segment (start 134.62 132.08) (end 131.318 132.08) (width 0.45) (layer F.Cu) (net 24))
 (segment (start 126.238 115.523483) (end 125.063833 114.349316) (width 0.45) (layer F.Cu) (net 24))
 (segment (start 126.238 127) (end 126.238 115.523483) (width 0.45) (layer F.Cu) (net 24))
 (segment (start 131.318 132.08) (end 126.238 127) (width 0.45) (layer F.Cu) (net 24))
 (segment (start 134.62 129.54) (end 131.318 129.54) (width 0.45) (layer F.Cu) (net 25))
 (segment (start 127.254 115.408113) (end 125.629518 113.783631) (width 0.45) (layer F.Cu) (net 25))
 (segment (start 127.254 125.476) (end 127.254 115.408113) (width 0.45) (layer F.Cu) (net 25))
 (segment (start 131.318 129.54) (end 127.254 125.476) (width 0.45) (layer F.Cu) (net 25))
 (segment (start 134.62 127) (end 131.318 127) (width 0.45) (layer F.Cu) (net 26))
 (segment (start 128.27 115.292742) (end 126.195204 113.217946) (width 0.45) (layer F.Cu) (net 26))
 (segment (start 128.27 123.952) (end 128.27 115.292742) (width 0.45) (layer F.Cu) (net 26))
 (segment (start 131.318 127) (end 128.27 123.952) (width 0.45) (layer F.Cu) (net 26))
 (segment (start 134.62 124.46) (end 131.318 124.46) (width 0.45) (layer F.Cu) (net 27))
 (segment (start 129.286 115.177371) (end 126.760889 112.65226) (width 0.45) (layer F.Cu) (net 27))
 (segment (start 129.286 122.428) (end 129.286 115.177371) (width 0.45) (layer F.Cu) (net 27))
 (segment (start 131.318 124.46) (end 129.286 122.428) (width 0.45) (layer F.Cu) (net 27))
 (segment (start 134.62 121.92) (end 132.146 121.92) (width 0.45) (layer F.Cu) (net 28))
 (segment (start 132.146 121.92) (end 131.826 121.6) (width 0.45) (layer F.Cu) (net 28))
 (segment (start 131.826 121.6) (end 130.744 121.6) (width 0.45) (layer F.Cu) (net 28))
 (segment (start 130.744 121.6) (end 130.302 121.158) (width 0.45) (layer F.Cu) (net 28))
 (segment (start 130.302 121.158) (end 130.302 115.062) (width 0.45) (layer F.Cu) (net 28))
 (segment (start 130.302 115.062) (end 127.326575 112.086575) (width 0.45) (layer F.Cu) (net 28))
 (segment (start 131.826 119.7) (end 131.826 118.618) (width 0.45) (layer F.Cu) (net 29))
 (segment (start 131.826 118.618) (end 131.318 118.11) (width 0.45) (layer F.Cu) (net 29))
 (segment (start 131.318 118.11) (end 131.318 114.946629) (width 0.45) (layer F.Cu) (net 29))
 (segment (start 131.318 114.946629) (end 127.89226 111.520889) (width 0.45) (layer F.Cu) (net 29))
 (segment (start 134.62 119.38) (end 132.146 119.38) (width 0.45) (layer F.Cu) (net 29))
 (segment (start 132.146 119.38) (end 131.826 119.7) (width 0.45) (layer F.Cu) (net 29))
 (segment (start 134.62 116.84) (end 133.096 116.84) (width 0.45) (layer F.Cu) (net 30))
 (segment (start 132.334 114.831258) (end 128.457946 110.955204) (width 0.45) (layer F.Cu) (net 30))
 (segment (start 132.334 116.078) (end 132.334 114.831258) (width 0.45) (layer F.Cu) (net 30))
 (segment (start 133.096 116.84) (end 132.334 116.078) (width 0.45) (layer F.Cu) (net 30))
 (segment (start 134.62 114.3) (end 132.842 114.3) (width 0.45) (layer F.Cu) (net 31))
 (segment (start 132.842 114.3) (end 129.023631 110.481631) (width 0.45) (layer F.Cu) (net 31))
 (segment (start 129.023631 110.481631) (end 129.023631 110.389518) (width 0.45) (layer F.Cu) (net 31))
 (segment (start 134.62 111.76) (end 131.525483 111.76) (width 0.45) (layer F.Cu) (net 32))
 (segment (start 131.525483 111.76) (end 129.589316 109.823833) (width 0.45) (layer F.Cu) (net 32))
 (segment (start 134.62 109.22) (end 132.588 109.22) (width 0.45) (layer F.Cu) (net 33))
 (segment (start 130.878854 109.982) (end 130.155002 109.258148) (width 0.45) (layer F.Cu) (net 33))
 (segment (start 131.826 109.982) (end 130.878854 109.982) (width 0.45) (layer F.Cu) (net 33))
 (segment (start 132.588 109.22) (end 131.826 109.982) (width 0.45) (layer F.Cu) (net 33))
 (segment (start 134.62 106.68) (end 132.588 106.68) (width 0.45) (layer F.Cu) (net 34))
 (segment (start 130.878854 105.918) (end 130.155002 106.641852) (width 0.45) (layer F.Cu) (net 34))
 (segment (start 131.826 105.918) (end 130.878854 105.918) (width 0.45) (layer F.Cu) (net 34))
 (segment (start 132.588 106.68) (end 131.826 105.918) (width 0.45) (layer F.Cu) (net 34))
 (segment (start 134.62 104.14) (end 131.525483 104.14) (width 0.45) (layer F.Cu) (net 35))
 (segment (start 131.525483 104.14) (end 129.589316 106.076167) (width 0.45) (layer F.Cu) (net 35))
 (segment (start 134.62 101.6) (end 132.934113 101.6) (width 0.45) (layer F.Cu) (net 36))
 (segment (start 132.934113 101.6) (end 129.023631 105.510482) (width 0.45) (layer F.Cu) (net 36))
 (segment (start 134.62 99.06) (end 133.096 99.06) (width 0.45) (layer F.Cu) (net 37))
 (segment (start 132.334 101.068742) (end 128.457946 104.944796) (width 0.45) (layer F.Cu) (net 37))
 (segment (start 132.334 99.822) (end 132.334 101.068742) (width 0.45) (layer F.Cu) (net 37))
 (segment (start 133.096 99.06) (end 132.334 99.822) (width 0.45) (layer F.Cu) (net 37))
 (segment (start 134.62 96.52) (end 132.08 96.52) (width 0.45) (layer F.Cu) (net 38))
 (segment (start 131.318 100.953371) (end 127.89226 104.379111) (width 0.45) (layer F.Cu) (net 38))
 (segment (start 131.318 97.282) (end 131.318 100.953371) (width 0.45) (layer F.Cu) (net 38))
 (segment (start 132.08 96.52) (end 131.318 97.282) (width 0.45) (layer F.Cu) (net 38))
 (segment (start 134.62 93.98) (end 132.146 93.98) (width 0.45) (layer F.Cu) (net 39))
 (segment (start 132.146 93.98) (end 131.826 93.66) (width 0.45) (layer F.Cu) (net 39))
 (segment (start 131.826 93.66) (end 131.13 93.66) (width 0.45) (layer F.Cu) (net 39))
 (segment (start 131.13 93.66) (end 130.302 94.488) (width 0.45) (layer F.Cu) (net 39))
 (segment (start 130.302 94.488) (end 130.302 94.996) (width 0.45) (layer F.Cu) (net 39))
 (segment (start 130.302 100.838) (end 127.326575 103.813425) (width 0.45) (layer F.Cu) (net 39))
 (segment (start 130.302 94.996) (end 130.302 100.838) (width 0.45) (layer F.Cu) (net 39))
 (segment (start 134.62 91.44) (end 132.146 91.44) (width 0.45) (layer F.Cu) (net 40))
 (segment (start 132.146 91.44) (end 131.826 91.76) (width 0.45) (layer F.Cu) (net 40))
 (segment (start 131.826 91.76) (end 130.49 91.76) (width 0.45) (layer F.Cu) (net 40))
 (segment (start 130.49 91.76) (end 129.286 92.964) (width 0.45) (layer F.Cu) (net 40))
 (segment (start 129.286 100.722629) (end 126.760889 103.24774) (width 0.45) (layer F.Cu) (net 40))
 (segment (start 129.286 92.964) (end 129.286 100.722629) (width 0.45) (layer F.Cu) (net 40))
 (segment (start 134.62 88.9) (end 131.445 88.9) (width 0.45) (layer F.Cu) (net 41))
 (segment (start 128.27 100.607258) (end 126.195204 102.682054) (width 0.45) (layer F.Cu) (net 41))
 (segment (start 128.27 92.075) (end 128.27 100.607258) (width 0.45) (layer F.Cu) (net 41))
 (segment (start 131.445 88.9) (end 128.27 92.075) (width 0.45) (layer F.Cu) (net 41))
 (segment (start 134.62 86.36) (end 131.318 86.36) (width 0.45) (layer F.Cu) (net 42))
 (segment (start 127.254 100.491887) (end 125.629518 102.116369) (width 0.45) (layer F.Cu) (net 42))
 (segment (start 127.254 90.424) (end 127.254 100.491887) (width 0.45) (layer F.Cu) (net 42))
 (segment (start 131.318 86.36) (end 127.254 90.424) (width 0.45) (layer F.Cu) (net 42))
 (segment (start 134.62 83.82) (end 131.318 83.82) (width 0.45) (layer F.Cu) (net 43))
 (segment (start 126.238 100.376517) (end 125.063833 101.550684) (width 0.45) (layer F.Cu) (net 43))
 (segment (start 126.238 88.9) (end 126.238 100.376517) (width 0.45) (layer F.Cu) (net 43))
 (segment (start 131.318 83.82) (end 126.238 88.9) (width 0.45) (layer F.Cu) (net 43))
 (segment (start 125.233099 100.076486) (end 125.222 100.33) (width 0.45) (layer F.Cu) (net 44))
 (segment (start 125.222217 87.375783) (end 125.233099 100.076486) (width 0.45) (layer F.Cu) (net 44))
 (segment (start 125.222 100.33) (end 124.498148 100.984998) (width 0.45) (layer F.Cu) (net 44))
 (segment (start 131.318 81.28) (end 125.222217 87.375783) (width 0.45) (layer F.Cu) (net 44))
 (segment (start 134.62 81.28) (end 131.318 81.28) (width 0.45) (layer F.Cu) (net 44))
 (segment (start 116.924 117.602) (end 116.924 115.347371) (width 0.45) (layer F.Cu) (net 45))
 (segment (start 116.924 115.347371) (end 119.619111 112.65226) (width 0.45) (layer F.Cu) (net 45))
 (segment (start 116.586 122.09) (end 116.586 117.94) (width 0.45) (layer F.Cu) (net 45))
 (segment (start 116.586 117.94) (end 116.924 117.602) (width 0.45) (layer F.Cu) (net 45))
 (segment (start 111.76 73.914) (end 119.888 73.914) (width 0.45) (layer F.Cu) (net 46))
 (segment (start 122.682 76.708) (end 122.682 82.804) (width 0.45) (layer F.Cu) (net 46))
 (segment (start 119.888 73.914) (end 122.682 76.708) (width 0.45) (layer F.Cu) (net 46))
 (segment (start 134.62 76.454) (end 133.604 76.454) (width 0.45) (layer F.Cu) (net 47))
 (segment (start 133.604 76.454) (end 132.334 75.184) (width 0.45) (layer F.Cu) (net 47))
 (segment (start 132.334 75.184) (end 127.508 75.184) (width 0.45) (layer F.Cu) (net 47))
 (segment (start 127.508 75.184) (end 125.222 77.47) (width 0.45) (layer F.Cu) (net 47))
 (segment (start 125.222 77.47) (end 125.222 82.804) (width 0.45) (layer F.Cu) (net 47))
 (segment (start 123.19 88.646) (end 123.19 87.376) (width 0.45) (layer F.Cu) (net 49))
 (segment (start 127.254 81.026) (end 126.492 80.264) (width 0.45) (layer F.Cu) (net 49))
 (segment (start 127.254 83.312) (end 127.254 81.026) (width 0.45) (layer F.Cu) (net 49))
 (segment (start 126.492 84.074) (end 127.254 83.312) (width 0.45) (layer F.Cu) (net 49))
 (segment (start 123.19 87.376) (end 126.492 84.074) (width 0.45) (layer F.Cu) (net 49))
 (segment (start 134.62 73.914) (end 126.746 73.914) (width 0.45) (layer F.Cu) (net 50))
 (segment (start 123.952 76.708) (end 123.952 80.264) (width 0.45) (layer F.Cu) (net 50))
 (segment (start 126.746 73.914) (end 123.952 76.708) (width 0.45) (layer F.Cu) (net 50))
 (segment (start 111.76 76.454) (end 113.538 76.454) (width 0.45) (layer F.Cu) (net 51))
 (segment (start 121.412 77.47) (end 121.412 80.264) (width 0.45) (layer F.Cu) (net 51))
 (segment (start 119.126 75.184) (end 121.412 77.47) (width 0.45) (layer F.Cu) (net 51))
 (segment (start 114.808 75.184) (end 119.126 75.184) (width 0.45) (layer F.Cu) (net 51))
 (segment (start 113.538 76.454) (end 114.808 75.184) (width 0.45) (layer F.Cu) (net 51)))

